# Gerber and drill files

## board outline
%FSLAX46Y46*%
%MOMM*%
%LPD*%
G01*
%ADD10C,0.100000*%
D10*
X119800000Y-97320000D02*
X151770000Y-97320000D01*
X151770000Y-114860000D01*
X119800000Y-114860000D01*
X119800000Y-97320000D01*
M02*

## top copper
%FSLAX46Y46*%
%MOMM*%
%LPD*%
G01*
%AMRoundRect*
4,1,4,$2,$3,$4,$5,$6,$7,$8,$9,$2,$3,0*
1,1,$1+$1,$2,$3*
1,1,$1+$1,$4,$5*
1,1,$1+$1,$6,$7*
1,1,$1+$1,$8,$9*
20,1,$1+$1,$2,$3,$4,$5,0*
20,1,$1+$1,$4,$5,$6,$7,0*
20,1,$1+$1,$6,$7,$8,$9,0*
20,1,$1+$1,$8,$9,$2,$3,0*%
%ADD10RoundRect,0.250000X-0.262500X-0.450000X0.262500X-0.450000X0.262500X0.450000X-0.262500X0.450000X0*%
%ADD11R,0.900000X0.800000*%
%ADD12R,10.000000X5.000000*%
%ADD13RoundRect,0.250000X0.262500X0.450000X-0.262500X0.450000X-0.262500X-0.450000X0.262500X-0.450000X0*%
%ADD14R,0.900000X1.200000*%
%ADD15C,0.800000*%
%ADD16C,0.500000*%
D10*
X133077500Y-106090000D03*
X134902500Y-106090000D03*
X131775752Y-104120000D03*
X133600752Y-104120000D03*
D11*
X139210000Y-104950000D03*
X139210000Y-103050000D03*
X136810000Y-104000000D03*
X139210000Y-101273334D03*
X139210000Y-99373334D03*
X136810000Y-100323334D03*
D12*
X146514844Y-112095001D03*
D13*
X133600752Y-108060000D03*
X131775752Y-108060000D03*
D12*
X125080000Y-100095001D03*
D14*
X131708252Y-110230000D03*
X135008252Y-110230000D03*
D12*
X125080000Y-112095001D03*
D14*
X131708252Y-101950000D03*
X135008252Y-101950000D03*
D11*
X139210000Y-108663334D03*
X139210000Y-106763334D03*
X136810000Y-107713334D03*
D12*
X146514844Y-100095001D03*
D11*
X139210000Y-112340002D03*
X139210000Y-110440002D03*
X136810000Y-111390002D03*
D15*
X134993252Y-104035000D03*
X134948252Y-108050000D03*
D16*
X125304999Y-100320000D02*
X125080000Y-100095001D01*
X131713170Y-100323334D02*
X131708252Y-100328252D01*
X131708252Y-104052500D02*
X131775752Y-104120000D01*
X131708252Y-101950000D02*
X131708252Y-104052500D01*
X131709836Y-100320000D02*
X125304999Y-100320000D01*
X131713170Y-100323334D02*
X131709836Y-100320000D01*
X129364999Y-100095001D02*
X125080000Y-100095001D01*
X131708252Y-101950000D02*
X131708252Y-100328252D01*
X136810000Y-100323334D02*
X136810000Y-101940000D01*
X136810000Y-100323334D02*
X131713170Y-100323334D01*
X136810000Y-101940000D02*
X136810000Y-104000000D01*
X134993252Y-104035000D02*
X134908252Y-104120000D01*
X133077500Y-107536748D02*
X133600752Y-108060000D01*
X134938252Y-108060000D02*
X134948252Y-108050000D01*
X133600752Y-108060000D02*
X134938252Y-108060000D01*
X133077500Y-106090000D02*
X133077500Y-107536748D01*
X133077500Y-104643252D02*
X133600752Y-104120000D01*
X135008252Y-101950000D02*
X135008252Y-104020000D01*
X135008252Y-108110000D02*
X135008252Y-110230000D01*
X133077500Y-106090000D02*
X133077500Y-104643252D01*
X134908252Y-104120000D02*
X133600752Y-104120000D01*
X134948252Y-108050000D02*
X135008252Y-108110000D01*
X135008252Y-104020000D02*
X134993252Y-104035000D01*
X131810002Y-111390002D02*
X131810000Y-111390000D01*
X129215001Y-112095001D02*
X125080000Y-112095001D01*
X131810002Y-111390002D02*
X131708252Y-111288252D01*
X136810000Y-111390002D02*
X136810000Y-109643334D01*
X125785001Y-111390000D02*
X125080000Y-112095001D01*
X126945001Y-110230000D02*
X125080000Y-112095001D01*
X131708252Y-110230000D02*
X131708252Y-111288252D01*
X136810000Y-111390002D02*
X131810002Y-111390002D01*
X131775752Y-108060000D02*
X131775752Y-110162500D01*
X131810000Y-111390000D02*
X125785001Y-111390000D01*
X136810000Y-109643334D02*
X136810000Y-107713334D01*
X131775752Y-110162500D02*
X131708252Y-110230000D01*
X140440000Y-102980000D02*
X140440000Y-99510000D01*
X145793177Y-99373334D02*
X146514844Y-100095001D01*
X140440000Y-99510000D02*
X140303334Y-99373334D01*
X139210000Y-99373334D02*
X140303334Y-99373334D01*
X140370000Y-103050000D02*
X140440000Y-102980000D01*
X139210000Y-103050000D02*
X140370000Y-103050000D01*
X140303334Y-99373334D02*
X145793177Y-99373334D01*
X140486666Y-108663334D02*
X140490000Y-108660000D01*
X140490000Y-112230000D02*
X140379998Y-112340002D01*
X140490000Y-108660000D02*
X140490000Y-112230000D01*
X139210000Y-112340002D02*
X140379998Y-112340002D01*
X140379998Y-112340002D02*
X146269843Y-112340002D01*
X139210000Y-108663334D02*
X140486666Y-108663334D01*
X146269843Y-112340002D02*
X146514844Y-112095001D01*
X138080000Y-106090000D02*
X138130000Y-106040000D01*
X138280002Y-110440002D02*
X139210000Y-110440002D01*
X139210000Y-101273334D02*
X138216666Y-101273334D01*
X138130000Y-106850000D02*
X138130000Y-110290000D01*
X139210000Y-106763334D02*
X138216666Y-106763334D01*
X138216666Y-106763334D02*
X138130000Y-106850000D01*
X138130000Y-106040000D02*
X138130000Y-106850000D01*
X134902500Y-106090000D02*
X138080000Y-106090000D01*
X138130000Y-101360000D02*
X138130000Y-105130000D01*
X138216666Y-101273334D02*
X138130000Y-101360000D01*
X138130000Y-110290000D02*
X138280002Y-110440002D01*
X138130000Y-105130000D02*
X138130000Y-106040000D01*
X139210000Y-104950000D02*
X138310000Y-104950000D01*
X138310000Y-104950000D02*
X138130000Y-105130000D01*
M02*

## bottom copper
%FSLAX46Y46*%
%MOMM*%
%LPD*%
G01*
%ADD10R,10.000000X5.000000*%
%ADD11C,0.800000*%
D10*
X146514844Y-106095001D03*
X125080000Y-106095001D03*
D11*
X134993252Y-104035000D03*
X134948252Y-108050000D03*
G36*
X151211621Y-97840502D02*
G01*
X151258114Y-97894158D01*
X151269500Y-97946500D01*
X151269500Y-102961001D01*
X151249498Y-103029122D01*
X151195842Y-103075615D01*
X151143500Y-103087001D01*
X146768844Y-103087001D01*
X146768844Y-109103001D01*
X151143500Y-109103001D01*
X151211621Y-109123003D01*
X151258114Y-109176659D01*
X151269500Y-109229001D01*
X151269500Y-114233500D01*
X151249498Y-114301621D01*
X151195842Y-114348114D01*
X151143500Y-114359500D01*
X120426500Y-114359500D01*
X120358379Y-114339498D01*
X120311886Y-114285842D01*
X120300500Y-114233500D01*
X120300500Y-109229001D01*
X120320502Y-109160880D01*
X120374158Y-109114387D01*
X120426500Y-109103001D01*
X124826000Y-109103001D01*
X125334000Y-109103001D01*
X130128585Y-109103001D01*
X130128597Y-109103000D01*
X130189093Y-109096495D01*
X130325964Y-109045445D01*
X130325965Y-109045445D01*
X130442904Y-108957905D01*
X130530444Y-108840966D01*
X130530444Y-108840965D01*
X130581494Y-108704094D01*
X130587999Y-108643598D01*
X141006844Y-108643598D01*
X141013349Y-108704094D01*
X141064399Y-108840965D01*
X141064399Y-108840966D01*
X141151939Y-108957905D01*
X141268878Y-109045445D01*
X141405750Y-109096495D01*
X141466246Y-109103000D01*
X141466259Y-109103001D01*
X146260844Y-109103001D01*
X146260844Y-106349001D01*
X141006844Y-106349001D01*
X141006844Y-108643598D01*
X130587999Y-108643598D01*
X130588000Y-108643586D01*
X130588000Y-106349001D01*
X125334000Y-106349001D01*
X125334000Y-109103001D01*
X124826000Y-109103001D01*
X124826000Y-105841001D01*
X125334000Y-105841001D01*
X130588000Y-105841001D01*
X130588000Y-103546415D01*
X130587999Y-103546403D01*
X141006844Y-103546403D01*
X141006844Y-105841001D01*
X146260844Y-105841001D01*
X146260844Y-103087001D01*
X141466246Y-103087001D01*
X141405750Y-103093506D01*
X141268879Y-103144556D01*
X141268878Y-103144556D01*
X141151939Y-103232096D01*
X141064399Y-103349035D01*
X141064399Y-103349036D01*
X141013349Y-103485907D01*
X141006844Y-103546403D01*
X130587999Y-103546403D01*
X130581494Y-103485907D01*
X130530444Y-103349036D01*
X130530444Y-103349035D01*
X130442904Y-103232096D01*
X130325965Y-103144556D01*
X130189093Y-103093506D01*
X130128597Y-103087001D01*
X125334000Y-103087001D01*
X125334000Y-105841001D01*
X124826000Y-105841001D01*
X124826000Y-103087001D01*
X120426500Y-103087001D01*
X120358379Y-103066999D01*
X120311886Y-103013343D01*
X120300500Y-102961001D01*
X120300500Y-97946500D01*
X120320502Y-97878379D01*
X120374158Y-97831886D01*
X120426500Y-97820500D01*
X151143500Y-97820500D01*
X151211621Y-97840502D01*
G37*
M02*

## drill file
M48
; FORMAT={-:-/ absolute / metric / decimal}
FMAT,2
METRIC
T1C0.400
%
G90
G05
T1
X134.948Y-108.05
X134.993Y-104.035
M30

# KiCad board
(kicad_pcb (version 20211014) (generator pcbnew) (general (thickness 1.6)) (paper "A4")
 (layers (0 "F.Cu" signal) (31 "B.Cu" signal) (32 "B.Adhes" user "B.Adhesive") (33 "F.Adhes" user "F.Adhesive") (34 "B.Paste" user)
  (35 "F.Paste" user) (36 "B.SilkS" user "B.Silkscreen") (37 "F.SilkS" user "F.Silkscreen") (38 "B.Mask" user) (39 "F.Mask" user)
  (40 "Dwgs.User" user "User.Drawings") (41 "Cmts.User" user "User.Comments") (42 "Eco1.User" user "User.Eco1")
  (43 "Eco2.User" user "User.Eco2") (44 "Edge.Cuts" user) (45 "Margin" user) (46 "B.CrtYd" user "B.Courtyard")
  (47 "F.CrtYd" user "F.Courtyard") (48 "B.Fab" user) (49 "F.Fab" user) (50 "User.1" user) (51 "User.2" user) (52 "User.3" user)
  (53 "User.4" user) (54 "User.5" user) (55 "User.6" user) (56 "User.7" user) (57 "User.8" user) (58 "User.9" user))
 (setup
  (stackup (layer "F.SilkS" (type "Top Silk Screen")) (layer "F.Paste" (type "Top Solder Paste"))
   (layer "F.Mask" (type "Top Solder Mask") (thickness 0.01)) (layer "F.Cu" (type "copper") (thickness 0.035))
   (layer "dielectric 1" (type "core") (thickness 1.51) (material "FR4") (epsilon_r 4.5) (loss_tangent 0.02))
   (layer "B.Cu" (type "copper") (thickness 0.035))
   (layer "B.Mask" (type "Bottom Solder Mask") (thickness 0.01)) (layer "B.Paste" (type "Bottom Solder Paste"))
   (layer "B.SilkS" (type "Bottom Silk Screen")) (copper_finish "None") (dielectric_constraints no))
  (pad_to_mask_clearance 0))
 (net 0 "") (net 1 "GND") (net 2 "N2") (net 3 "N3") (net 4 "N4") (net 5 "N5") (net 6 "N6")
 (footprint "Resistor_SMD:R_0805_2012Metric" (layer "F.Cu") (at 133.99 106.09)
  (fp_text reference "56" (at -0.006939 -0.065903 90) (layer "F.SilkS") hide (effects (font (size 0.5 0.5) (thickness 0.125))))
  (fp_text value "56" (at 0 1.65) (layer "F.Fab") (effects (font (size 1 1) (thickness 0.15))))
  (pad "1" smd roundrect locked (at -0.9125 0) (size 1.025 1.4) (layers "F.Cu" "F.Paste" "F.Mask") (roundrect_rratio 0.243902) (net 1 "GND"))
  (pad "2" smd roundrect locked (at 0.9125 0) (size 1.025 1.4) (layers "F.Cu" "F.Paste" "F.Mask") (roundrect_rratio 0.243902) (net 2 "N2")))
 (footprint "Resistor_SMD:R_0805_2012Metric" (layer "F.Cu") (at 132.688252 104.12)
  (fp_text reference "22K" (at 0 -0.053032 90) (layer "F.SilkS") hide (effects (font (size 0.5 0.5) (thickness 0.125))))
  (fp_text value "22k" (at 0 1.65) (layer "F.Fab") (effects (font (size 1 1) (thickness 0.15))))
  (pad "1" smd roundrect locked (at -0.9125 0) (size 1.025 1.4) (layers "F.Cu" "F.Paste" "F.Mask") (roundrect_rratio 0.243902) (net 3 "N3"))
  (pad "2" smd roundrect locked (at 0.9125 0) (size 1.025 1.4) (layers "F.Cu" "F.Paste" "F.Mask") (roundrect_rratio 0.243902) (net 1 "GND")))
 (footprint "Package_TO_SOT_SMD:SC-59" (layer "F.Cu") (at 138.01 104 180)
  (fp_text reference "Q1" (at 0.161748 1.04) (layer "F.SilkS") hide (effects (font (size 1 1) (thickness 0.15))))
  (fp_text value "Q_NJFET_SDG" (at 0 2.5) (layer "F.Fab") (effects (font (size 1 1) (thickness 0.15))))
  (pad "1" smd rect locked (at -1.2 -0.95 180) (size 0.9 0.8) (layers "F.Cu" "F.Paste" "F.Mask") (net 2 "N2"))
  (pad "2" smd rect locked (at -1.2 0.95 180) (size 0.9 0.8) (layers "F.Cu" "F.Paste" "F.Mask") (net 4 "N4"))
  (pad "3" smd rect locked (at 1.2 0 180) (size 0.9 0.8) (layers "F.Cu" "F.Paste" "F.Mask") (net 3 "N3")))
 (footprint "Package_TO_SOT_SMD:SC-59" (layer "F.Cu") (at 138.01 100.323334 180)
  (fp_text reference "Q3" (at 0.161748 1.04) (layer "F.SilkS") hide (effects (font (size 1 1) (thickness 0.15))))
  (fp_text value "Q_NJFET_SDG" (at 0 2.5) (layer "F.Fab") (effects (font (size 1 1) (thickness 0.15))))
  (pad "1" smd rect locked (at -1.2 -0.95 180) (size 0.9 0.8) (layers "F.Cu" "F.Paste" "F.Mask") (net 2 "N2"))
  (pad "2" smd rect locked (at -1.2 0.95 180) (size 0.9 0.8) (layers "F.Cu" "F.Paste" "F.Mask") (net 4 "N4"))
  (pad "3" smd rect locked (at 1.2 0 180) (size 0.9 0.8) (layers "F.Cu" "F.Paste" "F.Mask") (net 3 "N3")))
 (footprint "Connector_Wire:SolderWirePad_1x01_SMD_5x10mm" (layer "F.Cu") (at 146.514844 112.095001 90)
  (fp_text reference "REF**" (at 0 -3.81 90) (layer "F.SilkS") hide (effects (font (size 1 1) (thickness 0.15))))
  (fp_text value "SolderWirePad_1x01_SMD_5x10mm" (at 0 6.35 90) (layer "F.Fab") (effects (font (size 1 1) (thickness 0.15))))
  (pad "1" smd rect locked (at 0 0 90) (size 5 10) (layers "F.Cu" "F.Paste" "F.Mask") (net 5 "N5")))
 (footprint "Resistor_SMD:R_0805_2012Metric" (layer "F.Cu") (at 132.688252 108.06 180)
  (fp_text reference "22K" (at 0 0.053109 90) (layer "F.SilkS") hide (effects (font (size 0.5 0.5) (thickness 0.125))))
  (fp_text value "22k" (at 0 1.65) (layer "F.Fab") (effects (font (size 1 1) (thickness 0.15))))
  (pad "1" smd roundrect locked (at -0.9125 0 180) (size 1.025 1.4) (layers "F.Cu" "F.Paste" "F.Mask") (roundrect_rratio 0.243902)
   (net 1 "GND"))
  (pad "2" smd roundrect locked (at 0.9125 0 180) (size 1.025 1.4) (layers "F.Cu" "F.Paste" "F.Mask") (roundrect_rratio 0.243902)
   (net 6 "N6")))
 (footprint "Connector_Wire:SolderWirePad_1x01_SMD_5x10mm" (layer "F.Cu") (at 125.08 100.095001 90)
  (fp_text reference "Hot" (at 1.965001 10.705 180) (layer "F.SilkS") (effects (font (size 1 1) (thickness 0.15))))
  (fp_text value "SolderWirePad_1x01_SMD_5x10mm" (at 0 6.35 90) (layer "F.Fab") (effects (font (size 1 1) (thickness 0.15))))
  (pad "1" smd rect locked (at 0 0 90) (size 5 10) (layers "F.Cu" "F.Paste" "F.Mask") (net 3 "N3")))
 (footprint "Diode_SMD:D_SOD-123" (layer "F.Cu") (at 133.358252 110.23)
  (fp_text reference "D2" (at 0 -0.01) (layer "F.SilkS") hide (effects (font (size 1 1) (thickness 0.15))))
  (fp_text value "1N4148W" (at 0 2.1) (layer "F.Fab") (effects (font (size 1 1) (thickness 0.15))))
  (pad "1" smd rect locked (at -1.65 0) (size 0.9 1.2) (layers "F.Cu" "F.Paste" "F.Mask") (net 6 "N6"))
  (pad "2" smd rect locked (at 1.65 0) (size 0.9 1.2) (layers "F.Cu" "F.Paste" "F.Mask") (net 1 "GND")))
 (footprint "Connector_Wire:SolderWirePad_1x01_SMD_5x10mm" (layer "F.Cu") (at 125.08 112.095001 90)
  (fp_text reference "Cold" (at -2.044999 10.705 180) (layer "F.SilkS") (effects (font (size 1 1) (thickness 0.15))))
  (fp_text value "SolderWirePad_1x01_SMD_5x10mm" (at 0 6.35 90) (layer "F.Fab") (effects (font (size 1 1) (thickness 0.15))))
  (pad "1" smd rect locked (at 0 0 90) (size 5 10) (layers "F.Cu" "F.Paste" "F.Mask") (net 6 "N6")))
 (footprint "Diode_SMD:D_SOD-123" (layer "F.Cu") (at 133.358252 101.95)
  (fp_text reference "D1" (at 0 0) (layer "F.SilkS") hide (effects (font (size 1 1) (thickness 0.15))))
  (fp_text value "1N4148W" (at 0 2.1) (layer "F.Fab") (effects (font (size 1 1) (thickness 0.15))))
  (pad "1" smd rect locked (at -1.65 0) (size 0.9 1.2) (layers "F.Cu" "F.Paste" "F.Mask") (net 3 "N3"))
  (pad "2" smd rect locked (at 1.65 0) (size 0.9 1.2) (layers "F.Cu" "F.Paste" "F.Mask") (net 1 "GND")))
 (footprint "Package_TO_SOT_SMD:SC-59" (layer "F.Cu") (at 138.01 107.713334 180)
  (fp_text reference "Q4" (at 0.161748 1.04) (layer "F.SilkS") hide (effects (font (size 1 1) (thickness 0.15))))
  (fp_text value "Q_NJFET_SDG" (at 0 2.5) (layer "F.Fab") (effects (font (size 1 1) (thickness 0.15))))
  (pad "1" smd rect locked (at -1.2 -0.95 180) (size 0.9 0.8) (layers "F.Cu" "F.Paste" "F.Mask") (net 5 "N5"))
  (pad "2" smd rect locked (at -1.2 0.95 180) (size 0.9 0.8) (layers "F.Cu" "F.Paste" "F.Mask") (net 2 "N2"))
  (pad "3" smd rect locked (at 1.2 0 180) (size 0.9 0.8) (layers "F.Cu" "F.Paste" "F.Mask") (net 6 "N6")))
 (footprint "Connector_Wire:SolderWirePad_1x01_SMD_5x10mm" (layer "F.Cu") (at 146.514844 100.095001 90)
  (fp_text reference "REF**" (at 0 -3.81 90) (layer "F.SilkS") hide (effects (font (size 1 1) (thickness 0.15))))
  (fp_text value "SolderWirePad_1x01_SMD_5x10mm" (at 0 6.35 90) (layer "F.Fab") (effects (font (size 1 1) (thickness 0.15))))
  (pad "1" smd rect locked (at 0 0 90) (size 5 10) (layers "F.Cu" "F.Paste" "F.Mask") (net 4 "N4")))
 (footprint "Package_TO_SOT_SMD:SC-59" (layer "F.Cu") (at 138.01 111.390002 180)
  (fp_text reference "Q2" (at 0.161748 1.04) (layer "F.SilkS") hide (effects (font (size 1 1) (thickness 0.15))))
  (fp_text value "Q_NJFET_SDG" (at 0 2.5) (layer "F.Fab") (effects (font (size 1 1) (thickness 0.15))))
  (pad "1" smd rect locked (at -1.2 -0.95 180) (size 0.9 0.8) (layers "F.Cu" "F.Paste" "F.Mask") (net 5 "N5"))
  (pad "2" smd rect locked (at -1.2 0.95 180) (size 0.9 0.8) (layers "F.Cu" "F.Paste" "F.Mask") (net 2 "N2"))
  (pad "3" smd rect locked (at 1.2 0 180) (size 0.9 0.8) (layers "F.Cu" "F.Paste" "F.Mask") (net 6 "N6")))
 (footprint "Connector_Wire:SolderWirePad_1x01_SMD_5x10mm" (layer "B.Cu") (at 146.514844 106.095001 90)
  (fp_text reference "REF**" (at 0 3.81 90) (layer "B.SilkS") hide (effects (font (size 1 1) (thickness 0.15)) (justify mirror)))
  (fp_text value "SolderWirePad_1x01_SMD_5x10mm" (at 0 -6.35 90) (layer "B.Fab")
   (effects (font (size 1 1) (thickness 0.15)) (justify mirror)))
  (pad "1" smd rect locked (at 0 0 90) (size 5 10) (layers "B.Cu" "B.Paste" "B.Mask") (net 1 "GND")))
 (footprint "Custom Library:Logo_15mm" (layer "B.Cu") (at 135.48 105.88 90)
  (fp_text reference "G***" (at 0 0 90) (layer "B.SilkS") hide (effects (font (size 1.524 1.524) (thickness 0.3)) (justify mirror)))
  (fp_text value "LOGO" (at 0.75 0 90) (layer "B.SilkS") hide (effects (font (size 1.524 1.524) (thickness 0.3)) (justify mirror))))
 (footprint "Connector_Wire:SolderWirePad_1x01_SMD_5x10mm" (layer "B.Cu") (at 125.08 106.095001 90)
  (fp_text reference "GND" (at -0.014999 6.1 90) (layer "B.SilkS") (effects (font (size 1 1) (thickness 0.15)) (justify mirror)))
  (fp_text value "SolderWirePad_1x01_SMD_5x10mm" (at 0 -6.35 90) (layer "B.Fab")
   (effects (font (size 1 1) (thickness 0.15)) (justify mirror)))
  (pad "1" smd rect locked (at 0 0 90) (size 5 10) (layers "B.Cu" "B.Paste" "B.Mask") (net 1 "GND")))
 (gr_rect (start 151.77 114.86) (end 119.8 97.32) (layer "Edge.Cuts") (width 0.1) (fill none))
 (segment (start 125.304999 100.32) (end 125.08 100.095001) (width 0.5) (layer "F.Cu") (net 3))
 (segment (start 131.71317 100.323334) (end 131.708252 100.328252) (width 0.5) (layer "F.Cu") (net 3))
 (segment (start 131.708252 104.0525) (end 131.775752 104.12) (width 0.5) (layer "F.Cu") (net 3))
 (segment (start 131.708252 101.95) (end 131.708252 104.0525) (width 0.5) (layer "F.Cu") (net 3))
 (segment (start 131.709836 100.32) (end 125.304999 100.32) (width 0.5) (layer "F.Cu") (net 3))
 (segment (start 131.71317 100.323334) (end 131.709836 100.32) (width 0.5) (layer "F.Cu") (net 3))
 (segment (start 129.364999 100.095001) (end 125.08 100.095001) (width 0.5) (layer "F.Cu") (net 3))
 (segment (start 131.708252 101.95) (end 131.708252 100.328252) (width 0.5) (layer "F.Cu") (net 3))
 (segment (start 136.81 100.323334) (end 136.81 101.94) (width 0.5) (layer "F.Cu") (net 3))
 (segment (start 136.81 100.323334) (end 131.71317 100.323334) (width 0.5) (layer "F.Cu") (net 3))
 (segment (start 136.81 101.94) (end 136.81 104) (width 0.5) (layer "F.Cu") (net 3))
 (segment (start 134.993252 104.035) (end 134.908252 104.12) (width 0.5) (layer "F.Cu") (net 1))
 (segment (start 133.0775 107.536748) (end 133.600752 108.06) (width 0.5) (layer "F.Cu") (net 1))
 (segment (start 134.938252 108.06) (end 134.948252 108.05) (width 0.5) (layer "F.Cu") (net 1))
 (segment (start 133.600752 108.06) (end 134.938252 108.06) (width 0.5) (layer "F.Cu") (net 1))
 (segment (start 133.0775 106.09) (end 133.0775 107.536748) (width 0.5) (layer "F.Cu") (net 1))
 (segment (start 133.0775 104.643252) (end 133.600752 104.12) (width 0.5) (layer "F.Cu") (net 1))
 (segment (start 135.008252 101.95) (end 135.008252 104.02) (width 0.5) (layer "F.Cu") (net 1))
 (segment (start 135.008252 108.11) (end 135.008252 110.23) (width 0.5) (layer "F.Cu") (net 1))
 (segment (start 133.0775 106.09) (end 133.0775 104.643252) (width 0.5) (layer "F.Cu") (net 1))
 (segment (start 134.908252 104.12) (end 133.600752 104.12) (width 0.5) (layer "F.Cu") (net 1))
 (segment (start 134.948252 108.05) (end 135.008252 108.11) (width 0.5) (layer "F.Cu") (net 1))
 (segment (start 135.008252 104.02) (end 134.993252 104.035) (width 0.5) (layer "F.Cu") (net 1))
 (via (at 134.993252 104.035) (size 0.8) (drill 0.4) (layers "F.Cu" "B.Cu") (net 1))
 (via (at 134.948252 108.05) (size 0.8) (drill 0.4) (layers "F.Cu" "B.Cu") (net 1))
 (segment (start 131.810002 111.390002) (end 131.81 111.39) (width 0.5) (layer "F.Cu") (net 6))
 (segment (start 129.215001 112.095001) (end 125.08 112.095001) (width 0.5) (layer "F.Cu") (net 6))
 (segment (start 131.810002 111.390002) (end 131.708252 111.288252) (width 0.5) (layer "F.Cu") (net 6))
 (segment (start 136.81 111.390002) (end 136.81 109.643334) (width 0.5) (layer "F.Cu") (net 6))
 (segment (start 125.785001 111.39) (end 125.08 112.095001) (width 0.5) (layer "F.Cu") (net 6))
 (segment (start 126.945001 110.23) (end 125.08 112.095001) (width 0.5) (layer "F.Cu") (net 6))
 (segment (start 131.708252 110.23) (end 131.708252 111.288252) (width 0.5) (layer "F.Cu") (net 6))
 (segment (start 136.81 111.390002) (end 131.810002 111.390002) (width 0.5) (layer "F.Cu") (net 6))
 (segment (start 131.775752 108.06) (end 131.775752 110.1625) (width 0.5) (layer "F.Cu") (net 6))
 (segment (start 131.81 111.39) (end 125.785001 111.39) (width 0.5) (layer "F.Cu") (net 6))
 (segment (start 136.81 109.643334) (end 136.81 107.713334) (width 0.5) (layer "F.Cu") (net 6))
 (segment (start 131.775752 110.1625) (end 131.708252 110.23) (width 0.5) (layer "F.Cu") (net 6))
 (segment (start 140.44 102.98) (end 140.44 99.51) (width 0.5) (layer "F.Cu") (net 4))
 (segment (start 145.793177 99.373334) (end 146.514844 100.095001) (width 0.5) (layer "F.Cu") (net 4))
 (segment (start 140.44 99.51) (end 140.303334 99.373334) (width 0.5) (layer "F.Cu") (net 4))
 (segment (start 139.21 99.373334) (end 140.303334 99.373334) (width 0.5) (layer "F.Cu") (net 4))
 (segment (start 140.37 103.05) (end 140.44 102.98) (width 0.5) (layer "F.Cu") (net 4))
 (segment (start 139.21 103.05) (end 140.37 103.05) (width 0.5) (layer "F.Cu") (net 4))
 (segment (start 140.303334 99.373334) (end 145.793177 99.373334) (width 0.5) (layer "F.Cu") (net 4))
 (segment (start 140.486666 108.663334) (end 140.49 108.66) (width 0.5) (layer "F.Cu") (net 5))
 (segment (start 140.49 112.23) (end 140.379998 112.340002) (width 0.5) (layer "F.Cu") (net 5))
 (segment (start 140.49 108.66) (end 140.49 112.23) (width 0.5) (layer "F.Cu") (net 5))
 (segment (start 139.21 112.340002) (end 140.379998 112.340002) (width 0.5) (layer "F.Cu") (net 5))
 (segment (start 140.379998 112.340002) (end 146.269843 112.340002) (width 0.5) (layer "F.Cu") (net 5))
 (segment (start 139.21 108.663334) (end 140.486666 108.663334) (width 0.5) (layer "F.Cu") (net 5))
 (segment (start 146.269843 112.340002) (end 146.514844 112.095001) (width 0.5) (layer "F.Cu") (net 5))
 (segment (start 138.08 106.09) (end 138.13 106.04) (width 0.5) (layer "F.Cu") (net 2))
 (segment (start 138.280002 110.440002) (end 139.21 110.440002) (width 0.5) (layer "F.Cu") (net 2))
 (segment (start 139.21 101.273334) (end 138.216666 101.273334) (width 0.5) (layer "F.Cu") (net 2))
 (segment (start 138.13 106.85) (end 138.13 110.29) (width 0.5) (layer "F.Cu") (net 2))
 (segment (start 139.21 106.763334) (end 138.216666 106.763334) (width 0.5) (layer "F.Cu") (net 2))
 (segment (start 138.216666 106.763334) (end 138.13 106.85) (width 0.5) (layer "F.Cu") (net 2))
 (segment (start 138.13 106.04) (end 138.13 106.85) (width 0.5) (layer "F.Cu") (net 2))
 (segment (start 134.9025 106.09) (end 138.08 106.09) (width 0.5) (layer "F.Cu") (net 2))
 (segment (start 138.13 101.36) (end 138.13 105.13) (width 0.5) (layer "F.Cu") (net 2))
 (segment (start 138.216666 101.273334) (end 138.13 101.36) (width 0.5) (layer "F.Cu") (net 2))
 (segment (start 138.13 110.29) (end 138.280002 110.440002) (width 0.5) (layer "F.Cu") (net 2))
 (segment (start 138.13 105.13) (end 138.13 106.04) (width 0.5) (layer "F.Cu") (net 2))
 (segment (start 139.21 104.95) (end 138.31 104.95) (width 0.5) (layer "F.Cu") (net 2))
 (segment (start 138.31 104.95) (end 138.13 105.13) (width 0.5) (layer "F.Cu") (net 2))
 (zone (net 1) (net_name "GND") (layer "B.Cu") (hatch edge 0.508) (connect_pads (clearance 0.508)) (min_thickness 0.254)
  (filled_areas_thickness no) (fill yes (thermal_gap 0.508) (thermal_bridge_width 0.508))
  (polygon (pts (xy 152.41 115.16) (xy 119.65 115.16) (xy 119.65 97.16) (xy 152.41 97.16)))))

